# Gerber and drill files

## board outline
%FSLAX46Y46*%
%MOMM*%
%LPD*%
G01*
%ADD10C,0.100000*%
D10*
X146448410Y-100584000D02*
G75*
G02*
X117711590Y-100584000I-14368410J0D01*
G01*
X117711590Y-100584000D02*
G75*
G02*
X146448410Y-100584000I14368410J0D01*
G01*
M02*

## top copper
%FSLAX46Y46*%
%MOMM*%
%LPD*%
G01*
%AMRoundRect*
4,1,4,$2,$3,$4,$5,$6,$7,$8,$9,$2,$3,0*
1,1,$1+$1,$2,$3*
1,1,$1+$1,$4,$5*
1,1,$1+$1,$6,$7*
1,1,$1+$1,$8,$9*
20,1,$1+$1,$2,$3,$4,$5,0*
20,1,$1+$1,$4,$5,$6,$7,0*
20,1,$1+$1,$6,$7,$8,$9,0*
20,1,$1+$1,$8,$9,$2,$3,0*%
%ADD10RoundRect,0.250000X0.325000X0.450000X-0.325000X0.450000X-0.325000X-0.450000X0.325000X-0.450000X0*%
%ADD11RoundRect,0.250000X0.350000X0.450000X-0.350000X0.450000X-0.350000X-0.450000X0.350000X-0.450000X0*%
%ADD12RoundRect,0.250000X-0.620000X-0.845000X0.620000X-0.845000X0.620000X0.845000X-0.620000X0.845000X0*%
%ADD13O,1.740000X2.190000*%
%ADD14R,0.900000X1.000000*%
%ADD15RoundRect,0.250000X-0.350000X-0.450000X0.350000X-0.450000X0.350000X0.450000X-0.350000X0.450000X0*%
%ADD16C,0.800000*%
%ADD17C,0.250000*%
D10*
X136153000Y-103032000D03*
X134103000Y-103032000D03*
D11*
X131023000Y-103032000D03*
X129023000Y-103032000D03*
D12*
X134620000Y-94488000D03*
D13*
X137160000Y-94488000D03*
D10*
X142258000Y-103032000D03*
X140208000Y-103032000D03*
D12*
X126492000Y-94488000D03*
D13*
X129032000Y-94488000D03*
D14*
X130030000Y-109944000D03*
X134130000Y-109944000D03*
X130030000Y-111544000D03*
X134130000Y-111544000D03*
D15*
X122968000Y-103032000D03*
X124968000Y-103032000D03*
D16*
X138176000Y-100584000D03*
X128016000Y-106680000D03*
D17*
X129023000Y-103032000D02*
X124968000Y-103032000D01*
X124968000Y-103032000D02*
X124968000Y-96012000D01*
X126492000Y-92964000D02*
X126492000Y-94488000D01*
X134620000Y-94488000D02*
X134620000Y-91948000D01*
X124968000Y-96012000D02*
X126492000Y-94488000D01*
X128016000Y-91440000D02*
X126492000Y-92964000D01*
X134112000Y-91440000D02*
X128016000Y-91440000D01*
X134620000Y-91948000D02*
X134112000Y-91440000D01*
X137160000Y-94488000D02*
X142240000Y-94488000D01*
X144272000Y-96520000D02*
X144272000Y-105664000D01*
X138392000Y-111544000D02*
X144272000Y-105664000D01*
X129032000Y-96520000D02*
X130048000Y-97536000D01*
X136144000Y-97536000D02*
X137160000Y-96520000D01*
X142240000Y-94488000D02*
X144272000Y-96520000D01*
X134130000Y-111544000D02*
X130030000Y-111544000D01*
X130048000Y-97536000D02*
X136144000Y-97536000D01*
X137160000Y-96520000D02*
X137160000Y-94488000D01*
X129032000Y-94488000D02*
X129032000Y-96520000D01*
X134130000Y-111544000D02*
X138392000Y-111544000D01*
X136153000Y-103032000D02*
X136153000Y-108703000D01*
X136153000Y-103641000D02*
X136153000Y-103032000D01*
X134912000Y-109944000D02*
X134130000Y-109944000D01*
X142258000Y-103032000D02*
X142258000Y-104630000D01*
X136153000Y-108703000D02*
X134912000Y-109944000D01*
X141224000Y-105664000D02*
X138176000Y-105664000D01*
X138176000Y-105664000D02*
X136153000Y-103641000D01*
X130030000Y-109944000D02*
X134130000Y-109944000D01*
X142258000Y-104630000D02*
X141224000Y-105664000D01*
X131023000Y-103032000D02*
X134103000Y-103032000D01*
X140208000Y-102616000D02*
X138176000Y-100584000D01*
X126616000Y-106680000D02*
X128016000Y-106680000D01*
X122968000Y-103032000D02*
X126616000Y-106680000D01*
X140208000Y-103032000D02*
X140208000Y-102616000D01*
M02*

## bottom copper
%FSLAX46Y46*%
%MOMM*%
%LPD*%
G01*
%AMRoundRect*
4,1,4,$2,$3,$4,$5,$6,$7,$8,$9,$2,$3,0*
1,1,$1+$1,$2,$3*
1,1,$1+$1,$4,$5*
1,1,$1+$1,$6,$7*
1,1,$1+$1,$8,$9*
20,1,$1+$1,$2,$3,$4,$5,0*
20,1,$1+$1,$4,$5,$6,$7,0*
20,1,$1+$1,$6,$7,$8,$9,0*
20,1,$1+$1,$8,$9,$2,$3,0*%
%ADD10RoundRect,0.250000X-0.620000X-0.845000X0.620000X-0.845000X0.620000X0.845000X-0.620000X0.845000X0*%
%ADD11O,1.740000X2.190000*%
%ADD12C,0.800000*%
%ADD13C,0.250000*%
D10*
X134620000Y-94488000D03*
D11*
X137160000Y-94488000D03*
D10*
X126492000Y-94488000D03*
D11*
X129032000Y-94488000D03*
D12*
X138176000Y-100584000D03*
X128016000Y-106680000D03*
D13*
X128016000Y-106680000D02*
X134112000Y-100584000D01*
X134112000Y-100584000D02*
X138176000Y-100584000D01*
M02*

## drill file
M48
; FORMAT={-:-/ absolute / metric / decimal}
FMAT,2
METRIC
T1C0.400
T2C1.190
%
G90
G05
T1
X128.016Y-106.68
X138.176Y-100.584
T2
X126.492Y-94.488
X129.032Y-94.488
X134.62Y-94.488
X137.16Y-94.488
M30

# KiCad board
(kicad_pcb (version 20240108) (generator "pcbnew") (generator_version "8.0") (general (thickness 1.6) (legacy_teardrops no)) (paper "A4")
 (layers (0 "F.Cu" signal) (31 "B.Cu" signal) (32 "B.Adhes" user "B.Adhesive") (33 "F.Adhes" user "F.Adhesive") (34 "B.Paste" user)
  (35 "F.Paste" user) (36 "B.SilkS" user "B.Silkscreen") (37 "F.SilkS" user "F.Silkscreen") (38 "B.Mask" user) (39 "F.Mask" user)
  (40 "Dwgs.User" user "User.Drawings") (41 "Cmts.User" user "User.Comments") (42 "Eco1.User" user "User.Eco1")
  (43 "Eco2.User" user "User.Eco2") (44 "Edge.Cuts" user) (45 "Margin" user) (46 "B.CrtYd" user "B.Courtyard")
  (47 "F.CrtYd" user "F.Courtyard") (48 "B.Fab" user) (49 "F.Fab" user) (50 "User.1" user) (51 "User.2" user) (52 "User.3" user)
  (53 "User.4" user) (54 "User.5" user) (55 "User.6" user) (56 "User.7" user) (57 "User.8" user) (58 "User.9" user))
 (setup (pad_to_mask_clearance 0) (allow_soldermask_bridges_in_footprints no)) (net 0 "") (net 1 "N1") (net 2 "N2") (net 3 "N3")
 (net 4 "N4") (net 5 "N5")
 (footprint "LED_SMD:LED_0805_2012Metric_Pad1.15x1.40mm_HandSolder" (layer "F.Cu") (at 135.128 103.032 180)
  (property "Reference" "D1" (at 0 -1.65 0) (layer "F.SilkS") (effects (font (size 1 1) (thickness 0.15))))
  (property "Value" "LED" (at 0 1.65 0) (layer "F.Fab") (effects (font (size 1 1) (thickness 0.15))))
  (pad "1" smd roundrect (at -1.025 0 180) (size 1.15 1.4) (layers "F.Cu" "F.Paste" "F.Mask") (roundrect_rratio 0.217391) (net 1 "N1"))
  (pad "2" smd roundrect (at 1.025 0 180) (size 1.15 1.4) (layers "F.Cu" "F.Paste" "F.Mask") (roundrect_rratio 0.217391) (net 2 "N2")))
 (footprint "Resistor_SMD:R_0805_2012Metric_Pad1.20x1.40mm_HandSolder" (layer "F.Cu") (at 130.023 103.032 180)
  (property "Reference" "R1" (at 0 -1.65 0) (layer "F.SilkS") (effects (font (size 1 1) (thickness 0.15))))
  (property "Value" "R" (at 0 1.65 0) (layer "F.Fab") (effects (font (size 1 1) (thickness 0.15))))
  (pad "1" smd roundrect (at -1 0 180) (size 1.2 1.4) (layers "F.Cu" "F.Paste" "F.Mask") (roundrect_rratio 0.208333) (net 2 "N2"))
  (pad "2" smd roundrect (at 1 0 180) (size 1.2 1.4) (layers "F.Cu" "F.Paste" "F.Mask") (roundrect_rratio 0.208333) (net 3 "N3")))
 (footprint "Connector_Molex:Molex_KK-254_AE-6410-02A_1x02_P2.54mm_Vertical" (layer "F.Cu") (at 134.62 94.488)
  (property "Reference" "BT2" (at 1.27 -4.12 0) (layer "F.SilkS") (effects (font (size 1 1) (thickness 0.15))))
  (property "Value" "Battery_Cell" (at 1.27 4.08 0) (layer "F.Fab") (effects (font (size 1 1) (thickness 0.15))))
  (pad "1" thru_hole roundrect (at 0 0) (size 1.74 2.19) (drill 1.19) (layers "*.Cu" "*.Mask") (remove_unused_layers no)
   (roundrect_rratio 0.143678) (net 3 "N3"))
  (pad "2" thru_hole oval (at 2.54 0) (size 1.74 2.19) (drill 1.19) (layers "*.Cu" "*.Mask") (remove_unused_layers no) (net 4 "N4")))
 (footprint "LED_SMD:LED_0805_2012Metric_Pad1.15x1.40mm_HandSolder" (layer "F.Cu") (at 141.233 103.032 180)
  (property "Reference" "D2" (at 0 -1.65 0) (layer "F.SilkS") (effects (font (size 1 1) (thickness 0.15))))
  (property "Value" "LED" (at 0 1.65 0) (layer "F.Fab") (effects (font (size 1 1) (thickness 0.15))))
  (pad "1" smd roundrect (at -1.025 0 180) (size 1.15 1.4) (layers "F.Cu" "F.Paste" "F.Mask") (roundrect_rratio 0.217391) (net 1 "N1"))
  (pad "2" smd roundrect (at 1.025 0 180) (size 1.15 1.4) (layers "F.Cu" "F.Paste" "F.Mask") (roundrect_rratio 0.217391) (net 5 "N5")))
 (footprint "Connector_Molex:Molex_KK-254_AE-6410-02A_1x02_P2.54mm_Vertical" (layer "F.Cu") (at 126.492 94.488)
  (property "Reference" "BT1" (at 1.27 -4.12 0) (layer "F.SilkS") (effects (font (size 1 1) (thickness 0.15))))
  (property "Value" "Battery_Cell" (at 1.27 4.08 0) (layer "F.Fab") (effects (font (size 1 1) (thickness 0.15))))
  (pad "1" thru_hole roundrect (at 0 0) (size 1.74 2.19) (drill 1.19) (layers "*.Cu" "*.Mask") (remove_unused_layers no)
   (roundrect_rratio 0.143678) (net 3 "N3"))
  (pad "2" thru_hole oval (at 2.54 0) (size 1.74 2.19) (drill 1.19) (layers "*.Cu" "*.Mask") (remove_unused_layers no) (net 4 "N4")))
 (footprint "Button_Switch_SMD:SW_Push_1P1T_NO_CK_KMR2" (layer "F.Cu") (at 132.08 110.744)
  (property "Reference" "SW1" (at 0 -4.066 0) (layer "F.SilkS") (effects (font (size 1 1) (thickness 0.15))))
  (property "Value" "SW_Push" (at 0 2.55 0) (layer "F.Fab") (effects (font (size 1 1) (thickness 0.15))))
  (pad "1" smd rect (at -2.05 -0.8) (size 0.9 1) (layers "F.Cu" "F.Paste" "F.Mask") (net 1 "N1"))
  (pad "1" smd rect (at 2.05 -0.8) (size 0.9 1) (layers "F.Cu" "F.Paste" "F.Mask") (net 1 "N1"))
  (pad "2" smd rect (at -2.05 0.8) (size 0.9 1) (layers "F.Cu" "F.Paste" "F.Mask") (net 4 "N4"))
  (pad "2" smd rect (at 2.05 0.8) (size 0.9 1) (layers "F.Cu" "F.Paste" "F.Mask") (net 4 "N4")))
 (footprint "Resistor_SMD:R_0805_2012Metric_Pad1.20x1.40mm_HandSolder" (layer "F.Cu") (at 123.968 103.032)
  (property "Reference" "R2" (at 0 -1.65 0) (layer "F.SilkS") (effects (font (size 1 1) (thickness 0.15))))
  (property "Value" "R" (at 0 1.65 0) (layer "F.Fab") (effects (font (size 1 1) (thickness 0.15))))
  (pad "1" smd roundrect (at -1 0) (size 1.2 1.4) (layers "F.Cu" "F.Paste" "F.Mask") (roundrect_rratio 0.208333) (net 5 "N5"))
  (pad "2" smd roundrect (at 1 0) (size 1.2 1.4) (layers "F.Cu" "F.Paste" "F.Mask") (roundrect_rratio 0.208333) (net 3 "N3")))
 (gr_circle (center 132.08 100.584) (end 146.304 102.616) (stroke (width 0.1) (type default)) (fill none) (layer "Edge.Cuts"))
 (segment (start 129.023 103.032) (end 124.968 103.032) (width 0.25) (layer "F.Cu") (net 3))
 (segment (start 124.968 103.032) (end 124.968 96.012) (width 0.25) (layer "F.Cu") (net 3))
 (segment (start 126.492 92.964) (end 126.492 94.488) (width 0.25) (layer "F.Cu") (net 3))
 (segment (start 134.62 94.488) (end 134.62 91.948) (width 0.25) (layer "F.Cu") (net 3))
 (segment (start 124.968 96.012) (end 126.492 94.488) (width 0.25) (layer "F.Cu") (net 3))
 (segment (start 128.016 91.44) (end 126.492 92.964) (width 0.25) (layer "F.Cu") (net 3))
 (segment (start 134.112 91.44) (end 128.016 91.44) (width 0.25) (layer "F.Cu") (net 3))
 (segment (start 134.62 91.948) (end 134.112 91.44) (width 0.25) (layer "F.Cu") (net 3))
 (segment (start 137.16 94.488) (end 142.24 94.488) (width 0.25) (layer "F.Cu") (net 4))
 (segment (start 144.272 96.52) (end 144.272 105.664) (width 0.25) (layer "F.Cu") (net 4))
 (segment (start 138.392 111.544) (end 144.272 105.664) (width 0.25) (layer "F.Cu") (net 4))
 (segment (start 129.032 96.52) (end 130.048 97.536) (width 0.25) (layer "F.Cu") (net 4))
 (segment (start 136.144 97.536) (end 137.16 96.52) (width 0.25) (layer "F.Cu") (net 4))
 (segment (start 142.24 94.488) (end 144.272 96.52) (width 0.25) (layer "F.Cu") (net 4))
 (segment (start 134.13 111.544) (end 130.03 111.544) (width 0.25) (layer "F.Cu") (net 4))
 (segment (start 130.048 97.536) (end 136.144 97.536) (width 0.25) (layer "F.Cu") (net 4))
 (segment (start 137.16 96.52) (end 137.16 94.488) (width 0.25) (layer "F.Cu") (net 4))
 (segment (start 129.032 94.488) (end 129.032 96.52) (width 0.25) (layer "F.Cu") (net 4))
 (segment (start 134.13 111.544) (end 138.392 111.544) (width 0.25) (layer "F.Cu") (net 4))
 (segment (start 136.153 103.032) (end 136.153 108.703) (width 0.25) (layer "F.Cu") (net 1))
 (segment (start 136.153 103.641) (end 136.153 103.032) (width 0.25) (layer "F.Cu") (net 1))
 (segment (start 134.912 109.944) (end 134.13 109.944) (width 0.25) (layer "F.Cu") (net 1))
 (segment (start 142.258 103.032) (end 142.258 104.63) (width 0.25) (layer "F.Cu") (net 1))
 (segment (start 136.153 108.703) (end 134.912 109.944) (width 0.25) (layer "F.Cu") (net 1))
 (segment (start 141.224 105.664) (end 138.176 105.664) (width 0.25) (layer "F.Cu") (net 1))
 (segment (start 138.176 105.664) (end 136.153 103.641) (width 0.25) (layer "F.Cu") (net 1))
 (segment (start 130.03 109.944) (end 134.13 109.944) (width 0.25) (layer "F.Cu") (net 1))
 (segment (start 142.258 104.63) (end 141.224 105.664) (width 0.25) (layer "F.Cu") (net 1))
 (segment (start 131.023 103.032) (end 134.103 103.032) (width 0.25) (layer "F.Cu") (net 2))
 (segment (start 140.208 102.616) (end 138.176 100.584) (width 0.25) (layer "F.Cu") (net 5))
 (segment (start 126.616 106.68) (end 128.016 106.68) (width 0.25) (layer "F.Cu") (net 5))
 (segment (start 122.968 103.032) (end 126.616 106.68) (width 0.25) (layer "F.Cu") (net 5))
 (segment (start 140.208 103.032) (end 140.208 102.616) (width 0.25) (layer "F.Cu") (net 5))
 (via (at 138.176 100.584) (size 0.8) (drill 0.4) (layers "F.Cu" "B.Cu") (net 5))
 (via (at 128.016 106.68) (size 0.8) (drill 0.4) (layers "F.Cu" "B.Cu") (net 5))
 (segment (start 128.016 106.68) (end 134.112 100.584) (width 0.25) (layer "B.Cu") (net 5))
 (segment (start 134.112 100.584) (end 138.176 100.584) (width 0.25) (layer "B.Cu") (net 5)))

